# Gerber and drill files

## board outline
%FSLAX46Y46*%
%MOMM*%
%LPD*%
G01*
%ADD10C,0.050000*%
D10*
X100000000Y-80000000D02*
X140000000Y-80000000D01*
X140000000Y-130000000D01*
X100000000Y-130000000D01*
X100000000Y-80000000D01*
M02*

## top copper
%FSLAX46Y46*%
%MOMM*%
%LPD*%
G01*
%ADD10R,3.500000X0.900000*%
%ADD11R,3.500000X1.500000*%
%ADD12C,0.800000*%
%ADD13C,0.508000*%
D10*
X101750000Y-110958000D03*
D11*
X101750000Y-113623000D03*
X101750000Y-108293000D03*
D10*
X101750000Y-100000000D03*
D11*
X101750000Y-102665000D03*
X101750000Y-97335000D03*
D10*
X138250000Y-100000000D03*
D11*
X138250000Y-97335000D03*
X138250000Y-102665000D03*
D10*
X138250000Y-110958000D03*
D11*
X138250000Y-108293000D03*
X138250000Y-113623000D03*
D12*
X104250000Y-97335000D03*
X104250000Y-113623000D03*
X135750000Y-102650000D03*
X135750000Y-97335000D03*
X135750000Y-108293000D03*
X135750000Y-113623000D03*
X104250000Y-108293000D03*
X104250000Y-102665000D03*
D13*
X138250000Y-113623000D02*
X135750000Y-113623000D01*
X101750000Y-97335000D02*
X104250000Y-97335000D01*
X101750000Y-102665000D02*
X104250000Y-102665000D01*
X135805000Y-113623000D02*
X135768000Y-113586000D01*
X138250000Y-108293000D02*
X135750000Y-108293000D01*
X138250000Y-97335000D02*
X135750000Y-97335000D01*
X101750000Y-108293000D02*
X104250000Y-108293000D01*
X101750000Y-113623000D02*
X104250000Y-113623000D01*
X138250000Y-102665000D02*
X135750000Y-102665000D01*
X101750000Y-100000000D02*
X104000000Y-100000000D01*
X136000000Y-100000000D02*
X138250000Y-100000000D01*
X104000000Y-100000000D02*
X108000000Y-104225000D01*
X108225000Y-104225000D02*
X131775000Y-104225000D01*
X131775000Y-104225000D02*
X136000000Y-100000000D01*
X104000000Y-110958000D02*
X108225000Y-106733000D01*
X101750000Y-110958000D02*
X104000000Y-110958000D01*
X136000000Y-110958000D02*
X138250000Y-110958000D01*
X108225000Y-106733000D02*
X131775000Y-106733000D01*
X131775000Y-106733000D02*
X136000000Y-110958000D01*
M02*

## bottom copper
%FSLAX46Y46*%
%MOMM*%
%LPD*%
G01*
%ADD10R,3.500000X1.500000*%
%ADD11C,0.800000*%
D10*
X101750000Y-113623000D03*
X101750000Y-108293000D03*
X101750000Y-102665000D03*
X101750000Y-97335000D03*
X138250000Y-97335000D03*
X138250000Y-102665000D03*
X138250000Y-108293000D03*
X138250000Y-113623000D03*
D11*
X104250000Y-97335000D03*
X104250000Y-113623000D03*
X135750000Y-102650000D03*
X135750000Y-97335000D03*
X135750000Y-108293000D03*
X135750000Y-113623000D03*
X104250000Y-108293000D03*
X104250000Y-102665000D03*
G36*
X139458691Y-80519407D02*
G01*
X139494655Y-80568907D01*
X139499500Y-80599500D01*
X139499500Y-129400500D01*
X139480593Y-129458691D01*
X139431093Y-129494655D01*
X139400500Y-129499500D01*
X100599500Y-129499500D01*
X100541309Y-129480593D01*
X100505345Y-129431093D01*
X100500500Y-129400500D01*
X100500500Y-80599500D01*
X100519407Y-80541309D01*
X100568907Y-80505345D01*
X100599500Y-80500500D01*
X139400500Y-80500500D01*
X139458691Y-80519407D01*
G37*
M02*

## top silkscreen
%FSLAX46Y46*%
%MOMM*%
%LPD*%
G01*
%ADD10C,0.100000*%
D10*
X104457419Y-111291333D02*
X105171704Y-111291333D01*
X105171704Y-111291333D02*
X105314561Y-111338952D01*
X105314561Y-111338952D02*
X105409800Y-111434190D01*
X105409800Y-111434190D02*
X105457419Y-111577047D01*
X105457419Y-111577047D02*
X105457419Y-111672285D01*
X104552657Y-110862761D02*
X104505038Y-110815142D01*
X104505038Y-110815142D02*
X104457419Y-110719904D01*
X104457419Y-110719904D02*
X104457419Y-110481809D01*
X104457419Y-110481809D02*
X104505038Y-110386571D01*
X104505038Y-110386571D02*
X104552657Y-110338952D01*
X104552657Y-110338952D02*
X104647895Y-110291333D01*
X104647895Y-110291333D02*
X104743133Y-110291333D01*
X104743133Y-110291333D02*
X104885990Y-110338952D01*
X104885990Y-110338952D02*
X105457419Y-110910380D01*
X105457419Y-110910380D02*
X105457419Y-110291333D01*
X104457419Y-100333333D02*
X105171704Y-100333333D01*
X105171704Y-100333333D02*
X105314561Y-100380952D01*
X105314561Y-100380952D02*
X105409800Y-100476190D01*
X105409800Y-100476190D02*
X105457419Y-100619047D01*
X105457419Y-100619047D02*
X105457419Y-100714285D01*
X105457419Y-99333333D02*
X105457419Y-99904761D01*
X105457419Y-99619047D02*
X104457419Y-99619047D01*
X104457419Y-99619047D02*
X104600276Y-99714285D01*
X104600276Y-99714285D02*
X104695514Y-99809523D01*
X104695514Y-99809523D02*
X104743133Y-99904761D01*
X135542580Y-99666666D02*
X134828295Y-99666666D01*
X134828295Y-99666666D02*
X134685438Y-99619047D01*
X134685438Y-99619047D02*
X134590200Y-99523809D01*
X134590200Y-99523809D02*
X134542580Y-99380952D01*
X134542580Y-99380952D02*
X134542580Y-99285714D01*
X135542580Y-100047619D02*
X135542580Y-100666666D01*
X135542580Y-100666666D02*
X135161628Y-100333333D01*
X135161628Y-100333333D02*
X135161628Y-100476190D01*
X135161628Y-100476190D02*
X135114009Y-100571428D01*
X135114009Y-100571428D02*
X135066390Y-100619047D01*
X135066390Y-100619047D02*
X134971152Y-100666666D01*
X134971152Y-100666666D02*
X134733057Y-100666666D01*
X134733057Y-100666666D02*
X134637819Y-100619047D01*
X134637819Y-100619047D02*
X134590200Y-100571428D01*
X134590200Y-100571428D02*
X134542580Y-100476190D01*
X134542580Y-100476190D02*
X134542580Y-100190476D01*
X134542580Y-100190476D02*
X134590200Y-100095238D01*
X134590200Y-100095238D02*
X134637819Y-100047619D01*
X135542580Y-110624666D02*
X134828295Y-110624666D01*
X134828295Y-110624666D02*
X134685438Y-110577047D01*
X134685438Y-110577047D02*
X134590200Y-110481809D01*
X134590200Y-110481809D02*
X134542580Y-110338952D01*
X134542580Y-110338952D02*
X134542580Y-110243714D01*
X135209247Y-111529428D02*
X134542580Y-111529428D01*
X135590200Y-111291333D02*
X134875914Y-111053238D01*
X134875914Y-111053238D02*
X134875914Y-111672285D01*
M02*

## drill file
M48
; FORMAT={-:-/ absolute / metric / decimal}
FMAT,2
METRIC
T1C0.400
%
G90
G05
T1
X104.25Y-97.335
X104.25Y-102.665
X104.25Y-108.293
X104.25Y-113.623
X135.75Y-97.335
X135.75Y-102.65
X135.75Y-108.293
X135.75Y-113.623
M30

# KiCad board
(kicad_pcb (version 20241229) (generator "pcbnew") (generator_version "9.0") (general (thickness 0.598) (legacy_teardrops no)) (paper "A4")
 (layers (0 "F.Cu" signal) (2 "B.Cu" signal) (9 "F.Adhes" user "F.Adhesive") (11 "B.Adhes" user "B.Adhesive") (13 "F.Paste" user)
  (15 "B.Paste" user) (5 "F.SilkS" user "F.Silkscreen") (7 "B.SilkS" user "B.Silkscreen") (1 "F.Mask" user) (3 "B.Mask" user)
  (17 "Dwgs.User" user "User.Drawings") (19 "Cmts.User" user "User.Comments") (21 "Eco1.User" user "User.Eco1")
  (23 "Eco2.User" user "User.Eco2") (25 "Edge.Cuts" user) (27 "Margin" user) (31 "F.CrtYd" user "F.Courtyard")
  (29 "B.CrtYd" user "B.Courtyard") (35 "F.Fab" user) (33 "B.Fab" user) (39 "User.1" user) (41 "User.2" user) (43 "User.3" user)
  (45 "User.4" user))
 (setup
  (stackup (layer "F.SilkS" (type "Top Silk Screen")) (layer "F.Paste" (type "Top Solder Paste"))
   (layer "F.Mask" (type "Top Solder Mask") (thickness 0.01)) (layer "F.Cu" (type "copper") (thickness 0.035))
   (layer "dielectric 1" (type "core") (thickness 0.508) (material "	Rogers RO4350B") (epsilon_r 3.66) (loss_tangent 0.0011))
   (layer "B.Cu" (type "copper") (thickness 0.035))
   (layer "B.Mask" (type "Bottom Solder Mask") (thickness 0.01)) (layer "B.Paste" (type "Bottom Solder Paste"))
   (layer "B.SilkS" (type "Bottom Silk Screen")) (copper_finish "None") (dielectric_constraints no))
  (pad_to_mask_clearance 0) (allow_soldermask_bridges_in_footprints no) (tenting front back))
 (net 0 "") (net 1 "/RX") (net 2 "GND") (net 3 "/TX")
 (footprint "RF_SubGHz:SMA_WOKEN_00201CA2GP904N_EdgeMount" (layer "F.Cu") (at 100 110.958 90)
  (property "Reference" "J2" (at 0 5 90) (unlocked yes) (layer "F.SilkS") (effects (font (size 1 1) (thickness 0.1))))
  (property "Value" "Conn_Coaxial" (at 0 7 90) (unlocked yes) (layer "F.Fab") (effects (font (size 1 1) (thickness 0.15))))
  (pad "1" smd rect (at 0 1.75 90) (size 0.9 3.5) (layers "F.Cu" "F.Mask") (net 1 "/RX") (thermal_bridge_angle 45))
  (pad "2" smd rect (at -2.665 1.75 90) (size 1.5 3.5) (layers "F.Cu" "F.Mask") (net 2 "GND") (thermal_bridge_angle 45))
  (pad "2" smd rect (at -2.665 1.75 90) (size 1.5 3.5) (layers "B.Cu" "B.Mask") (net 2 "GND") (thermal_bridge_angle 45))
  (pad "2" smd rect (at 2.665 1.75 90) (size 1.5 3.5) (layers "F.Cu" "F.Mask") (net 2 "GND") (thermal_bridge_angle 45))
  (pad "2" smd rect (at 2.665 1.75 90) (size 1.5 3.5) (layers "B.Cu" "B.Mask") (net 2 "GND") (thermal_bridge_angle 45)))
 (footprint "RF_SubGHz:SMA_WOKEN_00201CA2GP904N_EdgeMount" (layer "F.Cu") (at 100 100 90)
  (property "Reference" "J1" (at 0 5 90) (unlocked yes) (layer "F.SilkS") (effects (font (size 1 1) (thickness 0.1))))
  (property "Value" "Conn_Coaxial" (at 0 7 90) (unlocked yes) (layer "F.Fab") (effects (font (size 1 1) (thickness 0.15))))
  (pad "1" smd rect (at 0 1.75 90) (size 0.9 3.5) (layers "F.Cu" "F.Mask") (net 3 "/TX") (thermal_bridge_angle 45))
  (pad "2" smd rect (at -2.665 1.75 90) (size 1.5 3.5) (layers "F.Cu" "F.Mask") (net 2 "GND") (thermal_bridge_angle 45))
  (pad "2" smd rect (at -2.665 1.75 90) (size 1.5 3.5) (layers "B.Cu" "B.Mask") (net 2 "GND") (thermal_bridge_angle 45))
  (pad "2" smd rect (at 2.665 1.75 90) (size 1.5 3.5) (layers "F.Cu" "F.Mask") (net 2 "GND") (thermal_bridge_angle 45))
  (pad "2" smd rect (at 2.665 1.75 90) (size 1.5 3.5) (layers "B.Cu" "B.Mask") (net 2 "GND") (thermal_bridge_angle 45)))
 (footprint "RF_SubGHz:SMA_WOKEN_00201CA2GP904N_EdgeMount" (layer "F.Cu") (at 140 100 -90)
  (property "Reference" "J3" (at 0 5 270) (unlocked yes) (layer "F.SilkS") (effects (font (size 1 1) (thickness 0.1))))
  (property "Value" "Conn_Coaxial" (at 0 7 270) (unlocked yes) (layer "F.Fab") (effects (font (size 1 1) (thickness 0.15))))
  (pad "1" smd rect (at 0 1.75 270) (size 0.9 3.5) (layers "F.Cu" "F.Mask") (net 3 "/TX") (thermal_bridge_angle 45))
  (pad "2" smd rect (at -2.665 1.75 270) (size 1.5 3.5) (layers "F.Cu" "F.Mask") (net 2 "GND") (thermal_bridge_angle 45))
  (pad "2" smd rect (at -2.665 1.75 270) (size 1.5 3.5) (layers "B.Cu" "B.Mask") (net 2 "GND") (thermal_bridge_angle 45))
  (pad "2" smd rect (at 2.665 1.75 270) (size 1.5 3.5) (layers "F.Cu" "F.Mask") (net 2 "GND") (thermal_bridge_angle 45))
  (pad "2" smd rect (at 2.665 1.75 270) (size 1.5 3.5) (layers "B.Cu" "B.Mask") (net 2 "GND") (thermal_bridge_angle 45)))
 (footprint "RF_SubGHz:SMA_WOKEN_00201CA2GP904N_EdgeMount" (layer "F.Cu") (at 140 110.958 -90)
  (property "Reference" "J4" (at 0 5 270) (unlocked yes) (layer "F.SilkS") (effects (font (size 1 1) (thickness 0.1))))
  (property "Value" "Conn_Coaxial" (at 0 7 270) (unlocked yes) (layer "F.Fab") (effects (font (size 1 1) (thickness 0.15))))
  (pad "1" smd rect (at 0 1.75 270) (size 0.9 3.5) (layers "F.Cu" "F.Mask") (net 1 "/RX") (thermal_bridge_angle 45))
  (pad "2" smd rect (at -2.665 1.75 270) (size 1.5 3.5) (layers "F.Cu" "F.Mask") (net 2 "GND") (thermal_bridge_angle 45))
  (pad "2" smd rect (at -2.665 1.75 270) (size 1.5 3.5) (layers "B.Cu" "B.Mask") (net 2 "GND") (thermal_bridge_angle 45))
  (pad "2" smd rect (at 2.665 1.75 270) (size 1.5 3.5) (layers "F.Cu" "F.Mask") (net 2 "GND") (thermal_bridge_angle 45))
  (pad "2" smd rect (at 2.665 1.75 270) (size 1.5 3.5) (layers "B.Cu" "B.Mask") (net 2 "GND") (thermal_bridge_angle 45)))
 (gr_rect (start 100 80) (end 140 130) (stroke (width 0.05) (type solid)) (fill no) (layer "Edge.Cuts"))
 (segment (start 138.25 113.623) (end 135.75 113.623) (width 0.508) (layer "F.Cu") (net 2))
 (segment (start 101.75 97.335) (end 104.25 97.335) (width 0.508) (layer "F.Cu") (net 2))
 (segment (start 101.75 102.665) (end 104.25 102.665) (width 0.508) (layer "F.Cu") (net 2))
 (segment (start 135.805 113.623) (end 135.768 113.586) (width 0.508) (layer "F.Cu") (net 2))
 (segment (start 138.25 108.293) (end 135.75 108.293) (width 0.508) (layer "F.Cu") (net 2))
 (segment (start 138.25 97.335) (end 135.75 97.335) (width 0.508) (layer "F.Cu") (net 2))
 (segment (start 101.75 108.293) (end 104.25 108.293) (width 0.508) (layer "F.Cu") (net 2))
 (segment (start 101.75 113.623) (end 104.25 113.623) (width 0.508) (layer "F.Cu") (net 2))
 (segment (start 138.25 102.665) (end 135.75 102.665) (width 0.508) (layer "F.Cu") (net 2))
 (via (at 104.25 97.335) (size 0.8) (drill 0.4) (layers "F.Cu" "B.Cu") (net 2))
 (via (at 104.25 113.623) (size 0.8) (drill 0.4) (layers "F.Cu" "B.Cu") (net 2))
 (via (at 135.75 102.65) (size 0.8) (drill 0.4) (layers "F.Cu" "B.Cu") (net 2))
 (via (at 135.75 97.335) (size 0.8) (drill 0.4) (layers "F.Cu" "B.Cu") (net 2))
 (via (at 135.75 108.293) (size 0.8) (drill 0.4) (layers "F.Cu" "B.Cu") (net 2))
 (via (at 135.75 113.623) (size 0.8) (drill 0.4) (layers "F.Cu" "B.Cu") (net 2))
 (via (at 104.25 108.293) (size 0.8) (drill 0.4) (layers "F.Cu" "B.Cu") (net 2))
 (via (at 104.25 102.665) (size 0.8) (drill 0.4) (layers "F.Cu" "B.Cu") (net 2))
 (segment (start 101.75 100) (end 104 100) (width 0.508) (layer "F.Cu") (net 3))
 (segment (start 136 100) (end 138.25 100) (width 0.508) (layer "F.Cu") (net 3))
 (segment (start 104 100) (end 108 104.225) (width 0.508) (layer "F.Cu") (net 3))
 (segment (start 108.225 104.225) (end 131.775 104.225) (width 0.508) (layer "F.Cu") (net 3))
 (segment (start 131.775 104.225) (end 136 100) (width 0.508) (layer "F.Cu") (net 3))
 (segment (start 104 110.958) (end 108.225 106.733) (width 0.508) (layer "F.Cu") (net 1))
 (segment (start 101.75 110.958) (end 104 110.958) (width 0.508) (layer "F.Cu") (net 1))
 (segment (start 136 110.958) (end 138.25 110.958) (width 0.508) (layer "F.Cu") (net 1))
 (segment (start 108.225 106.733) (end 131.775 106.733) (width 0.508) (layer "F.Cu") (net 1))
 (segment (start 131.775 106.733) (end 136 110.958) (width 0.508) (layer "F.Cu") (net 1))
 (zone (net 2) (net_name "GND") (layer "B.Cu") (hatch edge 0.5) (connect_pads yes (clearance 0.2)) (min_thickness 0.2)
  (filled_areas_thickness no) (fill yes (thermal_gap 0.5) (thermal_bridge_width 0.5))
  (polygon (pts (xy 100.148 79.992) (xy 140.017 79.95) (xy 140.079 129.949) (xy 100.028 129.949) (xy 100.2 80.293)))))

